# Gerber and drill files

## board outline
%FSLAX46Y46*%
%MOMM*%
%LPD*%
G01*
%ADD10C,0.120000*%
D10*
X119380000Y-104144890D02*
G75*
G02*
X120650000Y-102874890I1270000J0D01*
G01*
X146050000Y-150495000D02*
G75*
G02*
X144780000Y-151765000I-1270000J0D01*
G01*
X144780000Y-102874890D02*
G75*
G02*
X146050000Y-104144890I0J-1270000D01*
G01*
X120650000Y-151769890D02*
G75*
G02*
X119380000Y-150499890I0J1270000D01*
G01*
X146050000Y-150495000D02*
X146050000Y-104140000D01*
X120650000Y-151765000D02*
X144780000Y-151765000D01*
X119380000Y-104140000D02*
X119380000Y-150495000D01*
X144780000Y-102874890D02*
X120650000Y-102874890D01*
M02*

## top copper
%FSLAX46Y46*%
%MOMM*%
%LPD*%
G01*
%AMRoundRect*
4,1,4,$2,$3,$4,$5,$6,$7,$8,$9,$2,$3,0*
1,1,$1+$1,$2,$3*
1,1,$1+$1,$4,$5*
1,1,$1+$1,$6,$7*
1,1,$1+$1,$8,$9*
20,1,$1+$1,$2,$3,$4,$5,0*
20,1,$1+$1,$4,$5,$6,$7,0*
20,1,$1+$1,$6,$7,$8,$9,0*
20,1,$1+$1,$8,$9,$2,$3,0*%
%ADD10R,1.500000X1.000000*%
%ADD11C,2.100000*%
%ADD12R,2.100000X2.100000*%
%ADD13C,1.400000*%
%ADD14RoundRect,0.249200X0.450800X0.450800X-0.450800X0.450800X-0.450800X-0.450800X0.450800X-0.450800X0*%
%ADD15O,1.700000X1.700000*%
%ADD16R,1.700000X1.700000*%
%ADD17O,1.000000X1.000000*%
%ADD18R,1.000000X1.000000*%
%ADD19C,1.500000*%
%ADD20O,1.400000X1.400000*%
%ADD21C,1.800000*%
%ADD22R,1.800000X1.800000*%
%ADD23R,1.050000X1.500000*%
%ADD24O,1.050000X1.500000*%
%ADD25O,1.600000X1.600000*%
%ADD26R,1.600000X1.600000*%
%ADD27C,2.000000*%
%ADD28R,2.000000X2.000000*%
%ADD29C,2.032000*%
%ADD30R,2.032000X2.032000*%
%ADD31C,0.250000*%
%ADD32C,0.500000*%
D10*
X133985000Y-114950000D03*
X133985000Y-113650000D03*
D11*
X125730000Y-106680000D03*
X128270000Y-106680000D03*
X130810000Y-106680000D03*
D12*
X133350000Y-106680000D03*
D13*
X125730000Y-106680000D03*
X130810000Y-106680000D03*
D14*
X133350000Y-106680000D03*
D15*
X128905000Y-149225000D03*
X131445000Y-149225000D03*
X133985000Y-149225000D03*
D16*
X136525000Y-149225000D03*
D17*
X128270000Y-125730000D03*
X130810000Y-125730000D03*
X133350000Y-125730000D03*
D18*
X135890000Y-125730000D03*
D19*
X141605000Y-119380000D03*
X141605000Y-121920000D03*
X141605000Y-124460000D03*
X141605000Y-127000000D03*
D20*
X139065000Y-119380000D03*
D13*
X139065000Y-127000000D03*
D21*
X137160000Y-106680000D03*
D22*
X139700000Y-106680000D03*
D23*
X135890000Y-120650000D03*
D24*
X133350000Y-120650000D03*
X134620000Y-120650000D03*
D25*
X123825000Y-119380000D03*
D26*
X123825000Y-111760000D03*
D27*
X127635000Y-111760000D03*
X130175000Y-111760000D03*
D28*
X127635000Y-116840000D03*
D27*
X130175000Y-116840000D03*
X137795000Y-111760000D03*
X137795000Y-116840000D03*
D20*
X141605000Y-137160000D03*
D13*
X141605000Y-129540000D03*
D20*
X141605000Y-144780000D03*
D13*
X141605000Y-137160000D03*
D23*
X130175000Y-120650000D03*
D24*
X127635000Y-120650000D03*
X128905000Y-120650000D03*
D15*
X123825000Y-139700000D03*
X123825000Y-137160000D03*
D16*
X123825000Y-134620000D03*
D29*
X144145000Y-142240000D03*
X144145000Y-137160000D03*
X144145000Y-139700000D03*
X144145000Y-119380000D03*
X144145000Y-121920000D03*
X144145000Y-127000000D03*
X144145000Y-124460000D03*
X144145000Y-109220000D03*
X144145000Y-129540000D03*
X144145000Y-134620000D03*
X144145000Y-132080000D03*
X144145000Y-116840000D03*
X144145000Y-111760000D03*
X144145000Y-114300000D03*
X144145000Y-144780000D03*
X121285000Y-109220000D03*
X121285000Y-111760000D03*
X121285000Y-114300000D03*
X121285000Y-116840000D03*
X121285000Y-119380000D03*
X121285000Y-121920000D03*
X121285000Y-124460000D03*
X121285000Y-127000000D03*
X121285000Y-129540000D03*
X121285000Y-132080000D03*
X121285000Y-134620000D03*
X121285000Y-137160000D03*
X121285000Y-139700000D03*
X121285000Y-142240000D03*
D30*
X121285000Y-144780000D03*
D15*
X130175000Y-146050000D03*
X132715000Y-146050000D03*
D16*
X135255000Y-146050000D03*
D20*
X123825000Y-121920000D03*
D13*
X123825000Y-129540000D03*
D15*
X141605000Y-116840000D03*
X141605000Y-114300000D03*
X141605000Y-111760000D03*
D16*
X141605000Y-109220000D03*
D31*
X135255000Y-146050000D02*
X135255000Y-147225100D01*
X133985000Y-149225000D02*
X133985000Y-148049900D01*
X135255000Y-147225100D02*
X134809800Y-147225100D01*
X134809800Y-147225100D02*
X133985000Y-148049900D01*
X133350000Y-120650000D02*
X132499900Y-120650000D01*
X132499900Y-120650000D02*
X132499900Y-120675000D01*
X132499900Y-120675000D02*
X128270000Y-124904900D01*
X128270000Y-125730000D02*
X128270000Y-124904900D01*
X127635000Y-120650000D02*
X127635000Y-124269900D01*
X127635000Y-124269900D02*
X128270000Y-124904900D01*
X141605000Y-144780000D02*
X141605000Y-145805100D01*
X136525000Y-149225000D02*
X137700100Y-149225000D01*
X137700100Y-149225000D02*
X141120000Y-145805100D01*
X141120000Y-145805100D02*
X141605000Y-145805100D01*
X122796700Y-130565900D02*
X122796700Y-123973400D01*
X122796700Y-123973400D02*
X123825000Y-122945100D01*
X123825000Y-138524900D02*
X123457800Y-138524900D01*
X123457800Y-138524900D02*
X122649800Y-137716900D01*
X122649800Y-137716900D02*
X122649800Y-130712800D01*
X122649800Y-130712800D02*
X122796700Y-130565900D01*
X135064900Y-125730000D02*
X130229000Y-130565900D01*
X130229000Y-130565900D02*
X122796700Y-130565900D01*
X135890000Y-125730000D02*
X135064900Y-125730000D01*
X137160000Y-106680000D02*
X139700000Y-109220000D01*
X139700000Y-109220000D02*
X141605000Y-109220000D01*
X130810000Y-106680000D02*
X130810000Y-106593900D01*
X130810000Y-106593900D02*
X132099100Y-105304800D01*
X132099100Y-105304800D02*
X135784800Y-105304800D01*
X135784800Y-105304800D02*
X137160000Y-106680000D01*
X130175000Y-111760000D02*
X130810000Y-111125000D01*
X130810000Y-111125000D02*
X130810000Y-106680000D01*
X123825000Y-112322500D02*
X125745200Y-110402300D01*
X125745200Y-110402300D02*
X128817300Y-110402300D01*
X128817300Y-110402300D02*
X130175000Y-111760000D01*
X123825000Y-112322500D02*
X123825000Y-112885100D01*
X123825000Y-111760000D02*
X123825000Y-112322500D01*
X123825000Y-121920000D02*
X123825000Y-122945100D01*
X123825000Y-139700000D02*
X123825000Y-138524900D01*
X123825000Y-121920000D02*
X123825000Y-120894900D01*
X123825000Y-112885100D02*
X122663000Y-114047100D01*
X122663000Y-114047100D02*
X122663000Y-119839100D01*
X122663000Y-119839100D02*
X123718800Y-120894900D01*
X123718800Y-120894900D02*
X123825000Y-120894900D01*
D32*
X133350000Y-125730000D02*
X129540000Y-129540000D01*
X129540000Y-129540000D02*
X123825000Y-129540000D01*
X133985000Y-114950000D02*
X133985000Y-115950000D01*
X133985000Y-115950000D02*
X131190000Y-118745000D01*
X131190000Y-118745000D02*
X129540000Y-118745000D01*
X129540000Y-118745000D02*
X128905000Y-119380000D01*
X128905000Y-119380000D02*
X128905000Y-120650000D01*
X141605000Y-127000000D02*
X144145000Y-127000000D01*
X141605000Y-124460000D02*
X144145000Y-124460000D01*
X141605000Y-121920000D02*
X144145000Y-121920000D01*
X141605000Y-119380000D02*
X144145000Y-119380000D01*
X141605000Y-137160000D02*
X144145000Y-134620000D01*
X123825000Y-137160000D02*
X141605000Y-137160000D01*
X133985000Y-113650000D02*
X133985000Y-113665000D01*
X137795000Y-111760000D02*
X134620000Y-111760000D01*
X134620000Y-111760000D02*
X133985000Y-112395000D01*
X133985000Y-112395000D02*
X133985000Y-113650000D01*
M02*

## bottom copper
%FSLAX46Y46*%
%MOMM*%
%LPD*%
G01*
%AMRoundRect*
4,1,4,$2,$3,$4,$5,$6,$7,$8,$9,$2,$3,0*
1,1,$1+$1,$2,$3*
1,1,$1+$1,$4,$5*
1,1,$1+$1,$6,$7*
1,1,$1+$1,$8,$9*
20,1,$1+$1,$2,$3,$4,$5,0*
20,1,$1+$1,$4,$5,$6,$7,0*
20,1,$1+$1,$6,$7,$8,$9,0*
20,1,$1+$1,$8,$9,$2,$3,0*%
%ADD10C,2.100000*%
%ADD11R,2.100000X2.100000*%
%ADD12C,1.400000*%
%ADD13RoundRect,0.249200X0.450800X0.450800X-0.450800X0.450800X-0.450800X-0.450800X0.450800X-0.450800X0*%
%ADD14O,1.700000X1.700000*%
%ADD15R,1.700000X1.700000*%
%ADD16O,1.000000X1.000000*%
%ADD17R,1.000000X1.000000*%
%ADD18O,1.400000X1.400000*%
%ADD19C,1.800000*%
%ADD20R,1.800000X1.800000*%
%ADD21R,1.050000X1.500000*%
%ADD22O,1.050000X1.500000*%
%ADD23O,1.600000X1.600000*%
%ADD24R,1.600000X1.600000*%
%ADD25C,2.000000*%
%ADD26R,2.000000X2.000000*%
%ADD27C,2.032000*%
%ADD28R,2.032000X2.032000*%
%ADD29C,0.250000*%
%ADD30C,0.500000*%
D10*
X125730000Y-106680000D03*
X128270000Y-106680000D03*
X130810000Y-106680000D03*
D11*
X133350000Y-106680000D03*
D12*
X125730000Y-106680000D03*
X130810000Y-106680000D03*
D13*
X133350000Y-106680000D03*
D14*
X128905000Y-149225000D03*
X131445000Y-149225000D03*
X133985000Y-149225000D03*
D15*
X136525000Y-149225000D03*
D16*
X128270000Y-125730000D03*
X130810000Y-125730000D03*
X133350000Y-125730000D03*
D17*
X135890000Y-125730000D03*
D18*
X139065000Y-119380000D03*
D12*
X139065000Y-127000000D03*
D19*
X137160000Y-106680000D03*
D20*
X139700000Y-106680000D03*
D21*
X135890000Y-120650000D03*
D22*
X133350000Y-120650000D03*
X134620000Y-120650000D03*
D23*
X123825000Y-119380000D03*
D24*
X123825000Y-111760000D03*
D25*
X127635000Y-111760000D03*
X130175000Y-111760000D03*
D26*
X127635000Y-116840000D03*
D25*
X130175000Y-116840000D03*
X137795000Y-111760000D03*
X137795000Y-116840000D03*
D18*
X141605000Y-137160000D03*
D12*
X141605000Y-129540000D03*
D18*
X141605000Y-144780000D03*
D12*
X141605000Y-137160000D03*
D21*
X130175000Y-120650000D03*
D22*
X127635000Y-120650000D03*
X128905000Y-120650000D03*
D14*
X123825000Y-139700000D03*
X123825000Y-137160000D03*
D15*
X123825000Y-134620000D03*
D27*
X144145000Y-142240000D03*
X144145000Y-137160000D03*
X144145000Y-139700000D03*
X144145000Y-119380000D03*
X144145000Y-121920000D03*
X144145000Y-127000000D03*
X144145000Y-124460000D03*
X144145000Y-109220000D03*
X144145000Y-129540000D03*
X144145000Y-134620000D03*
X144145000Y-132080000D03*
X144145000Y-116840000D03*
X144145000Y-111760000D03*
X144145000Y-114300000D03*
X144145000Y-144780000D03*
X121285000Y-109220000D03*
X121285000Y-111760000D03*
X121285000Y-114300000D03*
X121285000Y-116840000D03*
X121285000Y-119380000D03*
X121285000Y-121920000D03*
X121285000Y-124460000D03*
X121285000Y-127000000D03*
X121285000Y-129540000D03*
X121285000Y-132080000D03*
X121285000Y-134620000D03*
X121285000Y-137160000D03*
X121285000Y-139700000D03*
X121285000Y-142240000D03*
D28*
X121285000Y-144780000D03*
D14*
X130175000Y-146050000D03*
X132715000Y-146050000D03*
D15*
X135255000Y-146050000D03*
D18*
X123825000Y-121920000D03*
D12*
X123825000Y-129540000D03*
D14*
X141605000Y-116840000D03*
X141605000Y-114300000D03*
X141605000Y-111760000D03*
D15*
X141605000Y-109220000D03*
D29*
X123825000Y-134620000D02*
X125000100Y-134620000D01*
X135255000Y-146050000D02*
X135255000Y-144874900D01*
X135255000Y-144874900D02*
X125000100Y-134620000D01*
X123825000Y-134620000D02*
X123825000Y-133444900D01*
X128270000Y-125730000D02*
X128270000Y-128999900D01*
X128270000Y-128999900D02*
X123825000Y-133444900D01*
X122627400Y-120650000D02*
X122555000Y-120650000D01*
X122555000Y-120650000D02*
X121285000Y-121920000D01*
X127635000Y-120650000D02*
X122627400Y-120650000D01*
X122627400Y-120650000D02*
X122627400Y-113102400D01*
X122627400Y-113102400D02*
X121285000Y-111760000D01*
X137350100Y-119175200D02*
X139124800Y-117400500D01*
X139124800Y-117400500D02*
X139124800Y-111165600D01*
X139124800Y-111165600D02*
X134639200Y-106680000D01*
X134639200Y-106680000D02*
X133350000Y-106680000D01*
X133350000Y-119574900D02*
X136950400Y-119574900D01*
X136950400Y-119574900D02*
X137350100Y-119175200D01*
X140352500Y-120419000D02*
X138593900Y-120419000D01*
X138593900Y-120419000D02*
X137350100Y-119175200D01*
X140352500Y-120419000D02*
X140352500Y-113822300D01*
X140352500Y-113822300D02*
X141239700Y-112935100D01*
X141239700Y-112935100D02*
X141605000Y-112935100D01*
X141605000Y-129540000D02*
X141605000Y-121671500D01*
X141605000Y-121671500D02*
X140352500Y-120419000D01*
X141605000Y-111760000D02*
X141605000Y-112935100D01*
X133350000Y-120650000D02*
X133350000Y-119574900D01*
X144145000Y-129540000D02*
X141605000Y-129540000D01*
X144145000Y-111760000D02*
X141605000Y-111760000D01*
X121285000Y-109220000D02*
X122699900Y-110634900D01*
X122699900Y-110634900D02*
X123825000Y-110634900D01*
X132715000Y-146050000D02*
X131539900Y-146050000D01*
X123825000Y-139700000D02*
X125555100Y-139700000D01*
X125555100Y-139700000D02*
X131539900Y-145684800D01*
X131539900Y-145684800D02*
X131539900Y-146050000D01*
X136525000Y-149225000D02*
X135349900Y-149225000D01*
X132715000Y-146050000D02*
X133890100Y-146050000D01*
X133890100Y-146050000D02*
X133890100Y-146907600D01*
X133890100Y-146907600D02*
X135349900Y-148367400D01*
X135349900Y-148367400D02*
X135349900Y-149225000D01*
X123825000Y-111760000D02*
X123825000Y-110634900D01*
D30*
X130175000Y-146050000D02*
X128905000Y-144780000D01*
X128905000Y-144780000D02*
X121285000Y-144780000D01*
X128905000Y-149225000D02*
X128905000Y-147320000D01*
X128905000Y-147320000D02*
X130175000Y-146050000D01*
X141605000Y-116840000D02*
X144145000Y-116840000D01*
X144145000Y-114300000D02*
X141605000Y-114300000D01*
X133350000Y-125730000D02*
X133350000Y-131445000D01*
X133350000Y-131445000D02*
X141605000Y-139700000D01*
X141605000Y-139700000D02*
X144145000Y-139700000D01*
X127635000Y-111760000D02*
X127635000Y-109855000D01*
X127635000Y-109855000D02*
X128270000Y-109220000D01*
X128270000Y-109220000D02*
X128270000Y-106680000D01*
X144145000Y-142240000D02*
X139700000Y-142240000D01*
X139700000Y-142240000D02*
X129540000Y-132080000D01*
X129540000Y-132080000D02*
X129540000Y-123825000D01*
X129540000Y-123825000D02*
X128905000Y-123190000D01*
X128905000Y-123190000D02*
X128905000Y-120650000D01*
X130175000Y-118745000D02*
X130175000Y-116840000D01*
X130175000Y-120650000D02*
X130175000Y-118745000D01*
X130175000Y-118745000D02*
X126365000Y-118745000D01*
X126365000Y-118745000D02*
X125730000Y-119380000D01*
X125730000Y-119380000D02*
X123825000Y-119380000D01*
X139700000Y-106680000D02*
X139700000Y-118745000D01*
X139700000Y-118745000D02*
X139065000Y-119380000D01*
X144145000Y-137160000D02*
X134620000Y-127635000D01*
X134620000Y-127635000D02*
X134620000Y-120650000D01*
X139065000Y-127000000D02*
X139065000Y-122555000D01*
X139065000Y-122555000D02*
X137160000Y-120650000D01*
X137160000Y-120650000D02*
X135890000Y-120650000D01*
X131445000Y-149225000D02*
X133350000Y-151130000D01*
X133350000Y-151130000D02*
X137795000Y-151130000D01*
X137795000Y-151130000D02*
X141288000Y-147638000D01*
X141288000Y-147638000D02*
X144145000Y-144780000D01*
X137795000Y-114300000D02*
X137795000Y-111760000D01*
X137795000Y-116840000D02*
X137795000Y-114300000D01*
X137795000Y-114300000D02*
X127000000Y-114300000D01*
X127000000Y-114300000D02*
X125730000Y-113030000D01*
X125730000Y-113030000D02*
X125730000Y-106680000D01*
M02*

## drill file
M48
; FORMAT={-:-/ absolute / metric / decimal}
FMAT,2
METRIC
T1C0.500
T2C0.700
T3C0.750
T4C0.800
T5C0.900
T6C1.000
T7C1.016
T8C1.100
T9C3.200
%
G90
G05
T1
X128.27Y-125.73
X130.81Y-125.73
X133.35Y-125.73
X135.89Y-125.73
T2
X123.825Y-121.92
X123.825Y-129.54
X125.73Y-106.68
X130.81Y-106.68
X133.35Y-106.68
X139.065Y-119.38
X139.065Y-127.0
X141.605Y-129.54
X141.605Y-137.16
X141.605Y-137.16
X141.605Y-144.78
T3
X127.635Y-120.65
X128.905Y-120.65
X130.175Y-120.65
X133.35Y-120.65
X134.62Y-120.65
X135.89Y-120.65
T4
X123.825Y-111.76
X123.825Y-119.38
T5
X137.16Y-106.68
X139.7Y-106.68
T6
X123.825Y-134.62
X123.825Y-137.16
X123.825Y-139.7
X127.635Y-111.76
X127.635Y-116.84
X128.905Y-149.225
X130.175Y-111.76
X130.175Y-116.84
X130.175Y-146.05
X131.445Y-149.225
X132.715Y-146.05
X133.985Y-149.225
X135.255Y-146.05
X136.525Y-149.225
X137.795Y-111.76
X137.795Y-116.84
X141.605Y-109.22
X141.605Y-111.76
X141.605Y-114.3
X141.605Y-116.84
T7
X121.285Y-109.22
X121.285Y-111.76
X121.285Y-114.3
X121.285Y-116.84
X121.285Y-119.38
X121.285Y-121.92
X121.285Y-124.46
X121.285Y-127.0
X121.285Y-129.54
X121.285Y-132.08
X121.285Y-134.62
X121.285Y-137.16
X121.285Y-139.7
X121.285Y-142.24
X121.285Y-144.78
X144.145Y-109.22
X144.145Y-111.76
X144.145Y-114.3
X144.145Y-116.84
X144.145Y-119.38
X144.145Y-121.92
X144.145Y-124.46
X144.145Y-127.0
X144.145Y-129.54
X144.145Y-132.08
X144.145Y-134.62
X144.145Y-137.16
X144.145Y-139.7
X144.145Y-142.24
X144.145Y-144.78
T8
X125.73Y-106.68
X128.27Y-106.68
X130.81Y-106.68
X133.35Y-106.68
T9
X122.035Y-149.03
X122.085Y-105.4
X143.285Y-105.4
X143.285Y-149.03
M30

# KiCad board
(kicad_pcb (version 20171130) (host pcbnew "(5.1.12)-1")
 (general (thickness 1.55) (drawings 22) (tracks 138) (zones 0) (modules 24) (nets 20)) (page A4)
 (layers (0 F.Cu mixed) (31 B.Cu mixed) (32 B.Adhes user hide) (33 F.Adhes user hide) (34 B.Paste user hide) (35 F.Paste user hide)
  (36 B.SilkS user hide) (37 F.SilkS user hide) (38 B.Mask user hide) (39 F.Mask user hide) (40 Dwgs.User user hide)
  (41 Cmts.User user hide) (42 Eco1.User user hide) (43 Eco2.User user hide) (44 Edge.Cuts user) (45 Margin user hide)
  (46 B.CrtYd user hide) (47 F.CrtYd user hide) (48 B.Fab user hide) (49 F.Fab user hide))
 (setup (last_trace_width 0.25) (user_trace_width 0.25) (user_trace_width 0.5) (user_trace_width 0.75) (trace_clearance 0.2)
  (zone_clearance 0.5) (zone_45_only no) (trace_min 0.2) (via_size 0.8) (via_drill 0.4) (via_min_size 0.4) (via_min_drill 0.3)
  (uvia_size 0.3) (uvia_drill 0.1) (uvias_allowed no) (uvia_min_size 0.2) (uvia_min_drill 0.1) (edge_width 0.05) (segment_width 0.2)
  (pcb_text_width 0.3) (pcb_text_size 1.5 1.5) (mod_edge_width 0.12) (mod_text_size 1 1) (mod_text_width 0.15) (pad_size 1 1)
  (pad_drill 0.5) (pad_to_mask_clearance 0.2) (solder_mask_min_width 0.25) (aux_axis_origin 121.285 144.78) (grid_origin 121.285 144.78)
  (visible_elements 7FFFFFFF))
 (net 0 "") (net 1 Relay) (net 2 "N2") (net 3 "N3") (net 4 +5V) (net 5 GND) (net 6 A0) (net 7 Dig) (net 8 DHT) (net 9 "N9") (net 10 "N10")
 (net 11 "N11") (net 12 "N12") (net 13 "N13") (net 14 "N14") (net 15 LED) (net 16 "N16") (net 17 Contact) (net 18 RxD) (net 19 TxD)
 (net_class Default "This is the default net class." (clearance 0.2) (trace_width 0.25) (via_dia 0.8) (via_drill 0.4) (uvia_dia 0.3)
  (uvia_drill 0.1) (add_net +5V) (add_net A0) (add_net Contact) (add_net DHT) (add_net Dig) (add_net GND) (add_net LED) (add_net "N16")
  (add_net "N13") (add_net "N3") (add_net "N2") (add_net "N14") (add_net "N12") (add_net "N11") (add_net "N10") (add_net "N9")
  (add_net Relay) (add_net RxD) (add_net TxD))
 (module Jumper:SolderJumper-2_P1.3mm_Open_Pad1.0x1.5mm (layer F.Cu) (at 133.985 114.3 90)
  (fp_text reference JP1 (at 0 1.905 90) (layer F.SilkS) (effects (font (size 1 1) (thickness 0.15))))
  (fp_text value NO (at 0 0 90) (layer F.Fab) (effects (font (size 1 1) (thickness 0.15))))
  (pad 1 smd rect (at -0.65 0 90) (size 1 1.5) (layers F.Cu F.Mask) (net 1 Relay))
  (pad 2 smd rect (at 0.65 0 90) (size 1 1.5) (layers F.Cu F.Mask) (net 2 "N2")))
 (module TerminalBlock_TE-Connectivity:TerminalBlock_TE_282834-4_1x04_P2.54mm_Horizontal (layer F.Cu) (at 133.35 106.68 180)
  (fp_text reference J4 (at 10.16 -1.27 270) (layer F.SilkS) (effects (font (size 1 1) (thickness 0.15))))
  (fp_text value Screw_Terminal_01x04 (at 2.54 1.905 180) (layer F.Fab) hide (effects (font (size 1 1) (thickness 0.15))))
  (pad 4 thru_hole circle (at 7.62 0 180) (size 2.1 2.1) (drill 1.1) (layers *.Cu *.Mask) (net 2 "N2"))
  (pad 3 thru_hole circle (at 5.08 0 180) (size 2.1 2.1) (drill 1.1) (layers *.Cu *.Mask) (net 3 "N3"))
  (pad 2 thru_hole circle (at 2.54 0 180) (size 2.1 2.1) (drill 1.1) (layers *.Cu *.Mask) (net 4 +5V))
  (pad 1 thru_hole rect (at 0 0 180) (size 2.1 2.1) (drill 1.1) (layers *.Cu *.Mask) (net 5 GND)))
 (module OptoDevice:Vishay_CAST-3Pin (layer F.Cu) (at 133.35 106.68 180)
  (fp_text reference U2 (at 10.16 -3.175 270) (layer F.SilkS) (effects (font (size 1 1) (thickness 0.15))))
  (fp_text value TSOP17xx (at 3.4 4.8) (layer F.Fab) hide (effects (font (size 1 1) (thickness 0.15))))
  (pad 3 thru_hole circle (at 7.62 0 180) (size 1.4 1.4) (drill 0.7) (layers *.Cu *.Mask) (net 2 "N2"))
  (pad 2 thru_hole circle (at 2.54 0 180) (size 1.4 1.4) (drill 0.7) (layers *.Cu *.Mask) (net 4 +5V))
  (pad 1 thru_hole roundrect (at 0 0 180) (size 1.4 1.4) (drill 0.7) (layers *.Cu *.Mask) (roundrect_rratio 0.178) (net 5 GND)))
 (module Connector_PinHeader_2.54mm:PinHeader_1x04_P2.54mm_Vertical (layer F.Cu) (at 136.525 149.225 270)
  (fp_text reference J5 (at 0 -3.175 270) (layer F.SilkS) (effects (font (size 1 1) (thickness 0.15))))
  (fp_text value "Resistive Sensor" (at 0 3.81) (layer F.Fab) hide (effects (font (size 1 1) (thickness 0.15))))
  (pad 4 thru_hole oval (at 0 7.62 270) (size 1.7 1.7) (drill 1) (layers *.Cu *.Mask) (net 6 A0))
  (pad 3 thru_hole oval (at 0 5.08 270) (size 1.7 1.7) (drill 1) (layers *.Cu *.Mask) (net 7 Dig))
  (pad 2 thru_hole oval (at 0 2.54 270) (size 1.7 1.7) (drill 1) (layers *.Cu *.Mask) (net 5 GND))
  (pad 1 thru_hole rect (at 0 0 270) (size 1.7 1.7) (drill 1) (layers *.Cu *.Mask) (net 4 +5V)))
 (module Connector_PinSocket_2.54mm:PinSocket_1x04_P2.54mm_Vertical (layer F.Cu) (at 135.89 125.73 270)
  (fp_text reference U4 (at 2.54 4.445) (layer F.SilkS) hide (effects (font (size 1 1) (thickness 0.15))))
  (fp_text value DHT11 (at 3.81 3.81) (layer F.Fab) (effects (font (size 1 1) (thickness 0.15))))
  (pad 4 thru_hole oval (at 0 7.62 270) (size 1 1) (drill 0.5) (layers *.Cu *.Mask) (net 5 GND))
  (pad 3 thru_hole oval (at 0 5.08 270) (size 1 1) (drill 0.5) (layers *.Cu *.Mask))
  (pad 2 thru_hole oval (at 0 2.54 270) (size 1 1) (drill 0.5) (layers *.Cu *.Mask) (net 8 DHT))
  (pad 1 thru_hole rect (at 0 0 270) (size 1 1) (drill 0.5) (layers *.Cu *.Mask) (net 4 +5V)))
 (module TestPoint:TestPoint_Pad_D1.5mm (layer F.Cu) (at 141.605 119.38)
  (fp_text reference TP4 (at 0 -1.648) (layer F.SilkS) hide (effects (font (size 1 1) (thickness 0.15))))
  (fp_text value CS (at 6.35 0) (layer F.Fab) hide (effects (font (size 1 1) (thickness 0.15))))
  (pad 1 smd circle (at 0 0) (size 1.5 1.5) (layers F.Cu F.Mask) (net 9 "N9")))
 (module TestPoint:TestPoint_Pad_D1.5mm (layer F.Cu) (at 141.605 121.92)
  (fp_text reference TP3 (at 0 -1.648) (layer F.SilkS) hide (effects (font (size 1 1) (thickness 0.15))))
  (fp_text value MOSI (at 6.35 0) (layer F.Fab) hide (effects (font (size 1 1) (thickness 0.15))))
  (pad 1 smd circle (at 0 0) (size 1.5 1.5) (layers F.Cu F.Mask) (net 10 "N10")))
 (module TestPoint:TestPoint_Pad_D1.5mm (layer F.Cu) (at 141.605 124.46)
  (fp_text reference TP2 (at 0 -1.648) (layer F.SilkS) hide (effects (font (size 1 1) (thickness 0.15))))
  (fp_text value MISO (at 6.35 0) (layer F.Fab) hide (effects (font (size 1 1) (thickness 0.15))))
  (pad 1 smd circle (at 0 0) (size 1.5 1.5) (layers F.Cu F.Mask) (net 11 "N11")))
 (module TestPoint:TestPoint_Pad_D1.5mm (layer F.Cu) (at 141.605 127)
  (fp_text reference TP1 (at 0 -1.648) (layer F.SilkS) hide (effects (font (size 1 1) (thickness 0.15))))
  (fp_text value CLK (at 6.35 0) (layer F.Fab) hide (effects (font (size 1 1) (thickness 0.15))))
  (pad 1 smd circle (at 0 0) (size 1.5 1.5) (layers F.Cu F.Mask) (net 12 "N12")))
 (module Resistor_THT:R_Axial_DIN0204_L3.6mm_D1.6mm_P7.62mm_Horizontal (layer F.Cu) (at 139.065 127 90)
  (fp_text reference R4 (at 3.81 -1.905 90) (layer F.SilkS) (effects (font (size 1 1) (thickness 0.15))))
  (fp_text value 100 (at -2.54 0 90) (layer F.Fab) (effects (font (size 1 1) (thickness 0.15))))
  (pad 2 thru_hole oval (at 7.62 0 90) (size 1.4 1.4) (drill 0.7) (layers *.Cu *.Mask) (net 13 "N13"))
  (pad 1 thru_hole circle (at 0 0 90) (size 1.4 1.4) (drill 0.7) (layers *.Cu *.Mask) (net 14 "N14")))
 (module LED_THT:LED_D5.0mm (layer F.Cu) (at 139.7 106.68 180)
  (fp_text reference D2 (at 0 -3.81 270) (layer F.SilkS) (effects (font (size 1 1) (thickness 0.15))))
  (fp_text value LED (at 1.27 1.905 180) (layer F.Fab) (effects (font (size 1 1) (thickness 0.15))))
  (pad 2 thru_hole circle (at 2.54 0 180) (size 1.8 1.8) (drill 0.9) (layers *.Cu *.Mask) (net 4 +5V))
  (pad 1 thru_hole rect (at 0 0 180) (size 1.8 1.8) (drill 0.9) (layers *.Cu *.Mask) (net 13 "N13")))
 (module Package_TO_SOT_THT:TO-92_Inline (layer F.Cu) (at 135.89 120.65 180)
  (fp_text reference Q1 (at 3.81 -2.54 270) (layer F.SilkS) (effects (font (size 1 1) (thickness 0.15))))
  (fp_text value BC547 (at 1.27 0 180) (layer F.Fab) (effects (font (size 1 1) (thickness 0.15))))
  (pad 1 thru_hole rect (at 0 0 180) (size 1.05 1.5) (drill 0.75) (layers *.Cu *.Mask) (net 14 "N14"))
  (pad 3 thru_hole oval (at 2.54 0 180) (size 1.05 1.5) (drill 0.75) (layers *.Cu *.Mask) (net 5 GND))
  (pad 2 thru_hole oval (at 1.27 0 180) (size 1.05 1.5) (drill 0.75) (layers *.Cu *.Mask) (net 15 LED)))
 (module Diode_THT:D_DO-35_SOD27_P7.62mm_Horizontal (layer F.Cu) (at 123.825 111.76 270)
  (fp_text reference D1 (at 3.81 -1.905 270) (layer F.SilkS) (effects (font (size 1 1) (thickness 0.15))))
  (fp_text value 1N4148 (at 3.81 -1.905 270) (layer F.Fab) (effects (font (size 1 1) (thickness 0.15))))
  (pad 2 thru_hole oval (at 7.62 0 270) (size 1.6 1.6) (drill 0.8) (layers *.Cu *.Mask) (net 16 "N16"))
  (pad 1 thru_hole rect (at 0 0 270) (size 1.6 1.6) (drill 0.8) (layers *.Cu *.Mask) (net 4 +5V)))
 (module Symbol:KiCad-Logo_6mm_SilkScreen (layer B.Cu) (at 131.445 135.255 90)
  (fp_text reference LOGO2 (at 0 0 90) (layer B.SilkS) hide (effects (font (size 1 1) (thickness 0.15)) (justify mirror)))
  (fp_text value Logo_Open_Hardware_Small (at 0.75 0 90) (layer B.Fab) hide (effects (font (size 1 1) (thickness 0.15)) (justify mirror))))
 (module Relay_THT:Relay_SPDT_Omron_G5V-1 (layer F.Cu) (at 127.635 116.84 90)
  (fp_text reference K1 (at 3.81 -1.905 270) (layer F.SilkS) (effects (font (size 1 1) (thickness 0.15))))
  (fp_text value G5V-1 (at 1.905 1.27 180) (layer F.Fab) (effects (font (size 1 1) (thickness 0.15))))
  (pad 10 thru_hole circle (at 5.08 0 90) (size 2 2) (drill 1) (layers *.Cu *.Mask) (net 3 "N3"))
  (pad 9 thru_hole circle (at 5.08 2.54 90) (size 2 2) (drill 1) (layers *.Cu *.Mask) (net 4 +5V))
  (pad 1 thru_hole rect (at 0 0 90) (size 2 2) (drill 1) (layers *.Cu *.Mask))
  (pad 2 thru_hole circle (at 0 2.54 90) (size 2 2) (drill 1) (layers *.Cu *.Mask) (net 16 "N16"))
  (pad 6 thru_hole circle (at 5.08 10.16 90) (size 2 2) (drill 1) (layers *.Cu *.Mask) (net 2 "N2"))
  (pad 5 thru_hole circle (at 0 10.16 90) (size 2 2) (drill 1) (layers *.Cu *.Mask) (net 2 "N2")))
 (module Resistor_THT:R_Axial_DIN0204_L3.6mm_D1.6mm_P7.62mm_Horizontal (layer F.Cu) (at 141.605 129.54 270)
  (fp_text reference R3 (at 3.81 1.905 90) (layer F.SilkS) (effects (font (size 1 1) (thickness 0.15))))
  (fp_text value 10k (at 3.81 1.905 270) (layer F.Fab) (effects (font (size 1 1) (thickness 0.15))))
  (pad 2 thru_hole oval (at 7.62 0 270) (size 1.4 1.4) (drill 0.7) (layers *.Cu *.Mask) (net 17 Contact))
  (pad 1 thru_hole circle (at 0 0 270) (size 1.4 1.4) (drill 0.7) (layers *.Cu *.Mask) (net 5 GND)))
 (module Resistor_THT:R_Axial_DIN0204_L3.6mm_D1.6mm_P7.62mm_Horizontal (layer F.Cu) (at 141.605 137.16 270)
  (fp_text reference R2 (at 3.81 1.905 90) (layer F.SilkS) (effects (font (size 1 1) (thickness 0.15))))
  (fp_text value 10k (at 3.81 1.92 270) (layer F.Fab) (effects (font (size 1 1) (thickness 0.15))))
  (pad 2 thru_hole oval (at 7.62 0 270) (size 1.4 1.4) (drill 0.7) (layers *.Cu *.Mask) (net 4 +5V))
  (pad 1 thru_hole circle (at 0 0 270) (size 1.4 1.4) (drill 0.7) (layers *.Cu *.Mask) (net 17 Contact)))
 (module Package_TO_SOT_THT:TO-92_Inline (layer F.Cu) (at 130.175 120.65 180)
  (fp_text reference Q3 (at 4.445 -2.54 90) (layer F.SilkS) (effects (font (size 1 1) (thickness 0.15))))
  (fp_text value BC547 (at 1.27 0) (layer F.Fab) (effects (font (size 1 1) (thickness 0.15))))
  (pad 1 thru_hole rect (at 0 0 180) (size 1.05 1.5) (drill 0.75) (layers *.Cu *.Mask) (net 16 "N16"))
  (pad 3 thru_hole oval (at 2.54 0 180) (size 1.05 1.5) (drill 0.75) (layers *.Cu *.Mask) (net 5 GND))
  (pad 2 thru_hole oval (at 1.27 0 180) (size 1.05 1.5) (drill 0.75) (layers *.Cu *.Mask) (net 1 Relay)))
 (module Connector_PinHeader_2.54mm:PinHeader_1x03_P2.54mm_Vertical (layer F.Cu) (at 123.825 134.62)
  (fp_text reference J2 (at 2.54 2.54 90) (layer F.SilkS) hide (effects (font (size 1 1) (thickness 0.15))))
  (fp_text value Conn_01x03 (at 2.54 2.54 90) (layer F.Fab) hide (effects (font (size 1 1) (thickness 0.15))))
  (pad 3 thru_hole oval (at 0 5.08) (size 1.7 1.7) (drill 1) (layers *.Cu *.Mask) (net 4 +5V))
  (pad 2 thru_hole oval (at 0 2.54) (size 1.7 1.7) (drill 1) (layers *.Cu *.Mask) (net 17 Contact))
  (pad 1 thru_hole rect (at 0 0) (size 1.7 1.7) (drill 1) (layers *.Cu *.Mask) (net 5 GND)))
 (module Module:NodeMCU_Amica (layer B.Cu) (at 121.285 144.78)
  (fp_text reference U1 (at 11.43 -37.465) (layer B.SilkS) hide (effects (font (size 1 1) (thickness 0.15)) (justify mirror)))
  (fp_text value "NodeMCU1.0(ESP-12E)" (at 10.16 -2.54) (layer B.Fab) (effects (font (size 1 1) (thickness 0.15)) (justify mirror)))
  (pad "" np_thru_hole circle (at 0.75 4.25) (size 3.2 3.2) (drill 3.2) (layers *.Cu *.Mask))
  (pad "" np_thru_hole circle (at 22 4.25) (size 3.2 3.2) (drill 3.2) (layers *.Cu *.Mask))
  (pad "" np_thru_hole circle (at 22 -39.38) (size 3.2 3.2) (drill 3.2) (layers *.Cu *.Mask))
  (pad "" np_thru_hole circle (at 0.8 -39.38) (size 3.2 3.2) (drill 3.2) (layers *.Cu *.Mask))
  (pad 29 thru_hole circle (at 22.86 -2.54) (size 2.032 2.032) (drill 1.016) (layers *.Cu *.Mask) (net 1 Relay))
  (pad 27 thru_hole circle (at 22.86 -7.62) (size 2.032 2.032) (drill 1.016) (layers *.Cu *.Mask) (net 15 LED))
  (pad 28 thru_hole circle (at 22.86 -5.08) (size 2.032 2.032) (drill 1.016) (layers *.Cu *.Mask) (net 8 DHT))
  (pad 20 thru_hole circle (at 22.86 -25.4) (size 2.032 2.032) (drill 1.016) (layers *.Cu *.Mask) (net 9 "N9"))
  (pad 21 thru_hole circle (at 22.86 -22.86) (size 2.032 2.032) (drill 1.016) (layers *.Cu *.Mask) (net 10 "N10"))
  (pad 23 thru_hole circle (at 22.86 -17.78) (size 2.032 2.032) (drill 1.016) (layers *.Cu *.Mask) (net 12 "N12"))
  (pad 22 thru_hole circle (at 22.86 -20.32) (size 2.032 2.032) (drill 1.016) (layers *.Cu *.Mask) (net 11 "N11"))
  (pad 16 thru_hole circle (at 22.86 -35.56) (size 2.032 2.032) (drill 1.016) (layers *.Cu *.Mask))
  (pad 24 thru_hole circle (at 22.86 -15.24) (size 2.032 2.032) (drill 1.016) (layers *.Cu *.Mask) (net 5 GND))
  (pad 26 thru_hole circle (at 22.86 -10.16) (size 2.032 2.032) (drill 1.016) (layers *.Cu *.Mask) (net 17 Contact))
  (pad 25 thru_hole circle (at 22.86 -12.7) (size 2.032 2.032) (drill 1.016) (layers *.Cu *.Mask))
  (pad 19 thru_hole circle (at 22.86 -27.94) (size 2.032 2.032) (drill 1.016) (layers *.Cu *.Mask) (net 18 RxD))
  (pad 17 thru_hole circle (at 22.86 -33.02) (size 2.032 2.032) (drill 1.016) (layers *.Cu *.Mask) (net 5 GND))
  (pad 18 thru_hole circle (at 22.86 -30.48) (size 2.032 2.032) (drill 1.016) (layers *.Cu *.Mask) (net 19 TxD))
  (pad 30 thru_hole circle (at 22.86 0) (size 2.032 2.032) (drill 1.016) (layers *.Cu *.Mask) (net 7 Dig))
  (pad 15 thru_hole circle (at 0 -35.56) (size 2.032 2.032) (drill 1.016) (layers *.Cu *.Mask) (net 4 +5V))
  (pad 14 thru_hole circle (at 0 -33.02) (size 2.032 2.032) (drill 1.016) (layers *.Cu *.Mask) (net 5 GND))
  (pad 13 thru_hole circle (at 0 -30.48) (size 2.032 2.032) (drill 1.016) (layers *.Cu *.Mask))
  (pad 12 thru_hole circle (at 0 -27.94) (size 2.032 2.032) (drill 1.016) (layers *.Cu *.Mask))
  (pad 11 thru_hole circle (at 0 -25.4) (size 2.032 2.032) (drill 1.016) (layers *.Cu *.Mask))
  (pad 10 thru_hole circle (at 0 -22.86) (size 2.032 2.032) (drill 1.016) (layers *.Cu *.Mask) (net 5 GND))
  (pad 9 thru_hole circle (at 0 -20.32) (size 2.032 2.032) (drill 1.016) (layers *.Cu *.Mask))
  (pad 8 thru_hole circle (at 0 -17.78) (size 2.032 2.032) (drill 1.016) (layers *.Cu *.Mask))
  (pad 7 thru_hole circle (at 0 -15.24) (size 2.032 2.032) (drill 1.016) (layers *.Cu *.Mask))
  (pad 6 thru_hole circle (at 0 -12.7) (size 2.032 2.032) (drill 1.016) (layers *.Cu *.Mask))
  (pad 5 thru_hole circle (at 0 -10.16) (size 2.032 2.032) (drill 1.016) (layers *.Cu *.Mask))
  (pad 4 thru_hole circle (at 0 -7.62) (size 2.032 2.032) (drill 1.016) (layers *.Cu *.Mask))
  (pad 3 thru_hole circle (at 0 -5.08) (size 2.032 2.032) (drill 1.016) (layers *.Cu *.Mask))
  (pad 2 thru_hole circle (at 0 -2.54) (size 2.032 2.032) (drill 1.016) (layers *.Cu *.Mask))
  (pad 1 thru_hole rect (at 0 0) (size 2.032 2.032) (drill 1.016) (layers *.Cu *.Mask) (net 6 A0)))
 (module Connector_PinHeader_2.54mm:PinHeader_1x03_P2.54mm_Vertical (layer F.Cu) (at 135.255 146.05 270)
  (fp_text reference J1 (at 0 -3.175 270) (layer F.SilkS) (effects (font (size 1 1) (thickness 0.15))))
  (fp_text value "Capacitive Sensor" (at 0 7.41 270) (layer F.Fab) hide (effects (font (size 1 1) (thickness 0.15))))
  (pad 3 thru_hole oval (at 0 5.08 270) (size 1.7 1.7) (drill 1) (layers *.Cu *.Mask) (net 6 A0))
  (pad 2 thru_hole oval (at 0 2.54 270) (size 1.7 1.7) (drill 1) (layers *.Cu *.Mask) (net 4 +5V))
  (pad 1 thru_hole rect (at 0 0 270) (size 1.7 1.7) (drill 1) (layers *.Cu *.Mask) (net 5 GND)))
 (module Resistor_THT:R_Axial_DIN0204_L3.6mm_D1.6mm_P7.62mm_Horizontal (layer F.Cu) (at 123.825 129.54 90)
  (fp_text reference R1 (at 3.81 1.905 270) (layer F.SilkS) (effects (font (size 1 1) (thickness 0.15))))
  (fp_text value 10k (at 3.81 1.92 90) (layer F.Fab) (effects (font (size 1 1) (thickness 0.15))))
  (pad 2 thru_hole oval (at 7.62 0 90) (size 1.4 1.4) (drill 0.7) (layers *.Cu *.Mask) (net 4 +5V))
  (pad 1 thru_hole circle (at 0 0 90) (size 1.4 1.4) (drill 0.7) (layers *.Cu *.Mask) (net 8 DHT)))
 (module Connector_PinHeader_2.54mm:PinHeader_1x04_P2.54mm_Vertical (layer F.Cu) (at 141.605 109.22)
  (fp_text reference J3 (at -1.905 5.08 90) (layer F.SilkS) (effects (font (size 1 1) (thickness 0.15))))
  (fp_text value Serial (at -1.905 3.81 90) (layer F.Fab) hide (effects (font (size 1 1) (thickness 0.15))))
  (pad 4 thru_hole oval (at 0 7.62) (size 1.7 1.7) (drill 1) (layers *.Cu *.Mask) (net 18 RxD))
  (pad 3 thru_hole oval (at 0 5.08) (size 1.7 1.7) (drill 1) (layers *.Cu *.Mask) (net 19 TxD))
  (pad 2 thru_hole oval (at 0 2.54) (size 1.7 1.7) (drill 1) (layers *.Cu *.Mask) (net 5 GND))
  (pad 1 thru_hole rect (at 0 0) (size 1.7 1.7) (drill 1) (layers *.Cu *.Mask) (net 4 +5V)))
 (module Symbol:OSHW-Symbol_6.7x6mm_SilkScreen (layer B.Cu) (at 137.795 142.24 90)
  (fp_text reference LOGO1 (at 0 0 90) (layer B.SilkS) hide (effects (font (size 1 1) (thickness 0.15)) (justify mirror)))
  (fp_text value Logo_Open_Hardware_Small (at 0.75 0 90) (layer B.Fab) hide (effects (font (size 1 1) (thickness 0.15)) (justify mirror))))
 (gr_arc (start 120.65 104.14489) (end 120.65 102.87489) (angle -90) (layer Edge.Cuts) (width 0.12))
 (gr_arc (start 144.78 150.495) (end 144.78 151.765) (angle -90) (layer Edge.Cuts) (width 0.12))
 (gr_arc (start 144.78 104.14489) (end 146.05 104.14489) (angle -90) (layer Edge.Cuts) (width 0.12))
 (gr_arc (start 120.65 150.49989) (end 119.38 150.49989) (angle -90) (layer Edge.Cuts) (width 0.12))
 (gr_line (start 146.05 150.495) (end 146.05 104.14) (layer Edge.Cuts) (width 0.12))
 (gr_line (start 120.65 151.765) (end 144.78 151.765) (layer Edge.Cuts) (width 0.12))
 (gr_line (start 119.38 104.14) (end 119.38 150.495) (layer Edge.Cuts) (width 0.12))
 (gr_line (start 144.78 102.87489) (end 120.65 102.87489) (layer Edge.Cuts) (width 0.12))
 (segment (start 123.825 134.62) (end 125.0001 134.62) (width 0.25) (layer B.Cu) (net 5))
 (segment (start 135.255 146.05) (end 135.255 144.8749) (width 0.25) (layer B.Cu) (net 5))
 (segment (start 135.255 144.8749) (end 125.0001 134.62) (width 0.25) (layer B.Cu) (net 5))
 (segment (start 123.825 134.62) (end 123.825 133.4449) (width 0.25) (layer B.Cu) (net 5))
 (segment (start 128.27 125.73) (end 128.27 128.9999) (width 0.25) (layer B.Cu) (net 5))
 (segment (start 128.27 128.9999) (end 123.825 133.4449) (width 0.25) (layer B.Cu) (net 5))
 (segment (start 135.255 146.05) (end 135.255 147.2251) (width 0.25) (layer F.Cu) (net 5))
 (segment (start 133.985 149.225) (end 133.985 148.0499) (width 0.25) (layer F.Cu) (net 5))
 (segment (start 135.255 147.2251) (end 134.8098 147.2251) (width 0.25) (layer F.Cu) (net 5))
 (segment (start 134.8098 147.2251) (end 133.985 148.0499) (width 0.25) (layer F.Cu) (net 5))
 (segment (start 122.6274 120.65) (end 122.555 120.65) (width 0.25) (layer B.Cu) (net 5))
 (segment (start 122.555 120.65) (end 121.285 121.92) (width 0.25) (layer B.Cu) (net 5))
 (segment (start 127.635 120.65) (end 122.6274 120.65) (width 0.25) (layer B.Cu) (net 5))
 (segment (start 122.6274 120.65) (end 122.6274 113.1024) (width 0.25) (layer B.Cu) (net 5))
 (segment (start 122.6274 113.1024) (end 121.285 111.76) (width 0.25) (layer B.Cu) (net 5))
 (segment (start 137.3501 119.1752) (end 139.1248 117.4005) (width 0.25) (layer B.Cu) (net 5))
 (segment (start 139.1248 117.4005) (end 139.1248 111.1656) (width 0.25) (layer B.Cu) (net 5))
 (segment (start 139.1248 111.1656) (end 134.6392 106.68) (width 0.25) (layer B.Cu) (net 5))
 (segment (start 134.6392 106.68) (end 133.35 106.68) (width 0.25) (layer B.Cu) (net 5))
 (segment (start 133.35 119.5749) (end 136.9504 119.5749) (width 0.25) (layer B.Cu) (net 5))
 (segment (start 136.9504 119.5749) (end 137.3501 119.1752) (width 0.25) (layer B.Cu) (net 5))
 (segment (start 140.3525 120.419) (end 138.5939 120.419) (width 0.25) (layer B.Cu) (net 5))
 (segment (start 138.5939 120.419) (end 137.3501 119.1752) (width 0.25) (layer B.Cu) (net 5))
 (segment (start 140.3525 120.419) (end 140.3525 113.8223) (width 0.25) (layer B.Cu) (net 5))
 (segment (start 140.3525 113.8223) (end 141.2397 112.9351) (width 0.25) (layer B.Cu) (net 5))
 (segment (start 141.2397 112.9351) (end 141.605 112.9351) (width 0.25) (layer B.Cu) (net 5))
 (segment (start 141.605 129.54) (end 141.605 121.6715) (width 0.25) (layer B.Cu) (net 5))
 (segment (start 141.605 121.6715) (end 140.3525 120.419) (width 0.25) (layer B.Cu) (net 5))
 (segment (start 141.605 111.76) (end 141.605 112.9351) (width 0.25) (layer B.Cu) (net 5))
 (segment (start 133.35 120.65) (end 133.35 119.5749) (width 0.25) (layer B.Cu) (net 5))
 (segment (start 144.145 129.54) (end 141.605 129.54) (width 0.25) (layer B.Cu) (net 5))
 (segment (start 133.35 120.65) (end 132.4999 120.65) (width 0.25) (layer F.Cu) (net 5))
 (segment (start 132.4999 120.65) (end 132.4999 120.675) (width 0.25) (layer F.Cu) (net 5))
 (segment (start 132.4999 120.675) (end 128.27 124.9049) (width 0.25) (layer F.Cu) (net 5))
 (segment (start 128.27 125.73) (end 128.27 124.9049) (width 0.25) (layer F.Cu) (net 5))
 (segment (start 127.635 120.65) (end 127.635 124.2699) (width 0.25) (layer F.Cu) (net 5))
 (segment (start 127.635 124.2699) (end 128.27 124.9049) (width 0.25) (layer F.Cu) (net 5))
 (segment (start 144.145 111.76) (end 141.605 111.76) (width 0.25) (layer B.Cu) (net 5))
 (segment (start 141.605 144.78) (end 141.605 145.8051) (width 0.25) (layer F.Cu) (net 4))
 (segment (start 136.525 149.225) (end 137.7001 149.225) (width 0.25) (layer F.Cu) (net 4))
 (segment (start 137.7001 149.225) (end 141.12 145.8051) (width 0.25) (layer F.Cu) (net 4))
 (segment (start 141.12 145.8051) (end 141.605 145.8051) (width 0.25) (layer F.Cu) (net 4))
 (segment (start 122.7967 130.5659) (end 122.7967 123.9734) (width 0.25) (layer F.Cu) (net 4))
 (segment (start 122.7967 123.9734) (end 123.825 122.9451) (width 0.25) (layer F.Cu) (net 4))
 (segment (start 123.825 138.5249) (end 123.4578 138.5249) (width 0.25) (layer F.Cu) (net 4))
 (segment (start 123.4578 138.5249) (end 122.6498 137.7169) (width 0.25) (layer F.Cu) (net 4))
 (segment (start 122.6498 137.7169) (end 122.6498 130.7128) (width 0.25) (layer F.Cu) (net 4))
 (segment (start 122.6498 130.7128) (end 122.7967 130.5659) (width 0.25) (layer F.Cu) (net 4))
 (segment (start 135.0649 125.73) (end 130.229 130.5659) (width 0.25) (layer F.Cu) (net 4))
 (segment (start 130.229 130.5659) (end 122.7967 130.5659) (width 0.25) (layer F.Cu) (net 4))
 (segment (start 135.89 125.73) (end 135.0649 125.73) (width 0.25) (layer F.Cu) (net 4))
 (segment (start 137.16 106.68) (end 139.7 109.22) (width 0.25) (layer F.Cu) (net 4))
 (segment (start 139.7 109.22) (end 141.605 109.22) (width 0.25) (layer F.Cu) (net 4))
 (segment (start 130.81 106.68) (end 130.81 106.5939) (width 0.25) (layer F.Cu) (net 4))
 (segment (start 130.81 106.5939) (end 132.0991 105.3048) (width 0.25) (layer F.Cu) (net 4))
 (segment (start 132.0991 105.3048) (end 135.7848 105.3048) (width 0.25) (layer F.Cu) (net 4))
 (segment (start 135.7848 105.3048) (end 137.16 106.68) (width 0.25) (layer F.Cu) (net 4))
 (segment (start 130.175 111.76) (end 130.81 111.125) (width 0.25) (layer F.Cu) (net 4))
 (segment (start 130.81 111.125) (end 130.81 106.68) (width 0.25) (layer F.Cu) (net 4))
 (segment (start 123.825 112.3225) (end 125.7452 110.4023) (width 0.25) (layer F.Cu) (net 4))
 (segment (start 125.7452 110.4023) (end 128.8173 110.4023) (width 0.25) (layer F.Cu) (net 4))
 (segment (start 128.8173 110.4023) (end 130.175 111.76) (width 0.25) (layer F.Cu) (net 4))
 (segment (start 123.825 112.3225) (end 123.825 112.8851) (width 0.25) (layer F.Cu) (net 4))
 (segment (start 123.825 111.76) (end 123.825 112.3225) (width 0.25) (layer F.Cu) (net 4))
 (segment (start 121.285 109.22) (end 122.6999 110.6349) (width 0.25) (layer B.Cu) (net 4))
 (segment (start 122.6999 110.6349) (end 123.825 110.6349) (width 0.25) (layer B.Cu) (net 4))
 (segment (start 123.825 121.92) (end 123.825 122.9451) (width 0.25) (layer F.Cu) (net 4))
 (segment (start 123.825 139.7) (end 123.825 138.5249) (width 0.25) (layer F.Cu) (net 4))
 (segment (start 123.825 121.92) (end 123.825 120.8949) (width 0.25) (layer F.Cu) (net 4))
 (segment (start 123.825 112.8851) (end 122.663 114.0471) (width 0.25) (layer F.Cu) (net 4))
 (segment (start 122.663 114.0471) (end 122.663 119.8391) (width 0.25) (layer F.Cu) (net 4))
 (segment (start 122.663 119.8391) (end 123.7188 120.8949) (width 0.25) (layer F.Cu) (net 4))
 (segment (start 123.7188 120.8949) (end 123.825 120.8949) (width 0.25) (layer F.Cu) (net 4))
 (segment (start 132.715 146.05) (end 131.5399 146.05) (width 0.25) (layer B.Cu) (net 4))
 (segment (start 123.825 139.7) (end 125.5551 139.7) (width 0.25) (layer B.Cu) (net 4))
 (segment (start 125.5551 139.7) (end 131.5399 145.6848) (width 0.25) (layer B.Cu) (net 4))
 (segment (start 131.5399 145.6848) (end 131.5399 146.05) (width 0.25) (layer B.Cu) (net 4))
 (segment (start 136.525 149.225) (end 135.3499 149.225) (width 0.25) (layer B.Cu) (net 4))
 (segment (start 132.715 146.05) (end 133.8901 146.05) (width 0.25) (layer B.Cu) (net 4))
 (segment (start 133.8901 146.05) (end 133.8901 146.9076) (width 0.25) (layer B.Cu) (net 4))
 (segment (start 133.8901 146.9076) (end 135.3499 148.3674) (width 0.25) (layer B.Cu) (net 4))
 (segment (start 135.3499 148.3674) (end 135.3499 149.225) (width 0.25) (layer B.Cu) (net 4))
 (segment (start 123.825 111.76) (end 123.825 110.6349) (width 0.25) (layer B.Cu) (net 4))
 (segment (start 130.175 146.05) (end 128.905 144.78) (width 0.5) (layer B.Cu) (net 6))
 (segment (start 128.905 144.78) (end 121.285 144.78) (width 0.5) (layer B.Cu) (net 6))
 (segment (start 128.905 149.225) (end 128.905 147.32) (width 0.5) (layer B.Cu) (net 6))
 (segment (start 128.905 147.32) (end 130.175 146.05) (width 0.5) (layer B.Cu) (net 6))
 (segment (start 141.605 116.84) (end 144.145 116.84) (width 0.5) (layer B.Cu) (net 18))
 (segment (start 144.145 114.3) (end 141.605 114.3) (width 0.5) (layer B.Cu) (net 19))
 (segment (start 133.35 125.73) (end 133.35 131.445) (width 0.5) (layer B.Cu) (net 8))
 (segment (start 133.35 131.445) (end 141.605 139.7) (width 0.5) (layer B.Cu) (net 8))
 (segment (start 141.605 139.7) (end 144.145 139.7) (width 0.5) (layer B.Cu) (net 8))
 (segment (start 133.35 125.73) (end 129.54 129.54) (width 0.5) (layer F.Cu) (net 8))
 (segment (start 129.54 129.54) (end 123.825 129.54) (width 0.5) (layer F.Cu) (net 8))
 (segment (start 127.635 111.76) (end 127.635 109.855) (width 0.5) (layer B.Cu) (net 3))
 (segment (start 127.635 109.855) (end 128.27 109.22) (width 0.5) (layer B.Cu) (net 3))
 (segment (start 128.27 109.22) (end 128.27 106.68) (width 0.5) (layer B.Cu) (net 3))
 (segment (start 133.985 114.95) (end 133.985 115.95) (width 0.5) (layer F.Cu) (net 1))
 (segment (start 133.985 115.95) (end 131.19 118.745) (width 0.5) (layer F.Cu) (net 1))
 (segment (start 131.19 118.745) (end 129.54 118.745) (width 0.5) (layer F.Cu) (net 1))
 (segment (start 129.54 118.745) (end 128.905 119.38) (width 0.5) (layer F.Cu) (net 1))
 (segment (start 128.905 119.38) (end 128.905 120.65) (width 0.5) (layer F.Cu) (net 1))
 (segment (start 144.145 142.24) (end 139.7 142.24) (width 0.5) (layer B.Cu) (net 1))
 (segment (start 139.7 142.24) (end 129.54 132.08) (width 0.5) (layer B.Cu) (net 1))
 (segment (start 129.54 132.08) (end 129.54 123.825) (width 0.5) (layer B.Cu) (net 1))
 (segment (start 129.54 123.825) (end 128.905 123.19) (width 0.5) (layer B.Cu) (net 1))
 (segment (start 128.905 123.19) (end 128.905 120.65) (width 0.5) (layer B.Cu) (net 1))
 (segment (start 130.175 118.745) (end 130.175 116.84) (width 0.5) (layer B.Cu) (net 16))
 (segment (start 130.175 120.65) (end 130.175 118.745) (width 0.5) (layer B.Cu) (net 16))
 (segment (start 130.175 118.745) (end 126.365 118.745) (width 0.5) (layer B.Cu) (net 16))
 (segment (start 126.365 118.745) (end 125.73 119.38) (width 0.5) (layer B.Cu) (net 16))
 (segment (start 125.73 119.38) (end 123.825 119.38) (width 0.5) (layer B.Cu) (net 16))
 (segment (start 139.7 106.68) (end 139.7 118.745) (width 0.5) (layer B.Cu) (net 13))
 (segment (start 139.7 118.745) (end 139.065 119.38) (width 0.5) (layer B.Cu) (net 13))
 (segment (start 144.145 137.16) (end 134.62 127.635) (width 0.5) (layer B.Cu) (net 15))
 (segment (start 134.62 127.635) (end 134.62 120.65) (width 0.5) (layer B.Cu) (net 15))
 (segment (start 139.065 127) (end 139.065 122.555) (width 0.5) (layer B.Cu) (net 14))
 (segment (start 139.065 122.555) (end 137.16 120.65) (width 0.5) (layer B.Cu) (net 14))
 (segment (start 137.16 120.65) (end 135.89 120.65) (width 0.5) (layer B.Cu) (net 14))
 (segment (start 141.605 127) (end 144.145 127) (width 0.5) (layer F.Cu) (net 12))
 (segment (start 141.605 124.46) (end 144.145 124.46) (width 0.5) (layer F.Cu) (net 11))
 (segment (start 141.605 121.92) (end 144.145 121.92) (width 0.5) (layer F.Cu) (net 10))
 (segment (start 141.605 119.38) (end 144.145 119.38) (width 0.5) (layer F.Cu) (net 9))
 (segment (start 131.445 149.225) (end 133.35 151.13) (width 0.5) (layer B.Cu) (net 7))
 (segment (start 133.35 151.13) (end 137.795 151.13) (width 0.5) (layer B.Cu) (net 7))
 (segment (start 137.795 151.13) (end 141.288 147.638) (width 0.5) (layer B.Cu) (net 7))
 (segment (start 141.288 147.638) (end 144.145 144.78) (width 0.5) (layer B.Cu) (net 7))
 (segment (start 141.605 137.16) (end 144.145 134.62) (width 0.5) (layer F.Cu) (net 17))
 (segment (start 123.825 137.16) (end 141.605 137.16) (width 0.5) (layer F.Cu) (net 17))
 (segment (start 137.795 114.3) (end 137.795 111.76) (width 0.5) (layer B.Cu) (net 2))
 (segment (start 137.795 116.84) (end 137.795 114.3) (width 0.5) (layer B.Cu) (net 2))
 (segment (start 133.985 113.65) (end 133.985 113.665) (width 0.5) (layer F.Cu) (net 2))
 (segment (start 137.795 111.76) (end 134.62 111.76) (width 0.5) (layer F.Cu) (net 2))
 (segment (start 134.62 111.76) (end 133.985 112.395) (width 0.5) (layer F.Cu) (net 2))
 (segment (start 133.985 112.395) (end 133.985 113.65) (width 0.5) (layer F.Cu) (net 2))
 (segment (start 137.795 114.3) (end 127 114.3) (width 0.5) (layer B.Cu) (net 2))
 (segment (start 127 114.3) (end 125.73 113.03) (width 0.5) (layer B.Cu) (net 2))
 (segment (start 125.73 113.03) (end 125.73 106.68) (width 0.5) (layer B.Cu) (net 2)))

